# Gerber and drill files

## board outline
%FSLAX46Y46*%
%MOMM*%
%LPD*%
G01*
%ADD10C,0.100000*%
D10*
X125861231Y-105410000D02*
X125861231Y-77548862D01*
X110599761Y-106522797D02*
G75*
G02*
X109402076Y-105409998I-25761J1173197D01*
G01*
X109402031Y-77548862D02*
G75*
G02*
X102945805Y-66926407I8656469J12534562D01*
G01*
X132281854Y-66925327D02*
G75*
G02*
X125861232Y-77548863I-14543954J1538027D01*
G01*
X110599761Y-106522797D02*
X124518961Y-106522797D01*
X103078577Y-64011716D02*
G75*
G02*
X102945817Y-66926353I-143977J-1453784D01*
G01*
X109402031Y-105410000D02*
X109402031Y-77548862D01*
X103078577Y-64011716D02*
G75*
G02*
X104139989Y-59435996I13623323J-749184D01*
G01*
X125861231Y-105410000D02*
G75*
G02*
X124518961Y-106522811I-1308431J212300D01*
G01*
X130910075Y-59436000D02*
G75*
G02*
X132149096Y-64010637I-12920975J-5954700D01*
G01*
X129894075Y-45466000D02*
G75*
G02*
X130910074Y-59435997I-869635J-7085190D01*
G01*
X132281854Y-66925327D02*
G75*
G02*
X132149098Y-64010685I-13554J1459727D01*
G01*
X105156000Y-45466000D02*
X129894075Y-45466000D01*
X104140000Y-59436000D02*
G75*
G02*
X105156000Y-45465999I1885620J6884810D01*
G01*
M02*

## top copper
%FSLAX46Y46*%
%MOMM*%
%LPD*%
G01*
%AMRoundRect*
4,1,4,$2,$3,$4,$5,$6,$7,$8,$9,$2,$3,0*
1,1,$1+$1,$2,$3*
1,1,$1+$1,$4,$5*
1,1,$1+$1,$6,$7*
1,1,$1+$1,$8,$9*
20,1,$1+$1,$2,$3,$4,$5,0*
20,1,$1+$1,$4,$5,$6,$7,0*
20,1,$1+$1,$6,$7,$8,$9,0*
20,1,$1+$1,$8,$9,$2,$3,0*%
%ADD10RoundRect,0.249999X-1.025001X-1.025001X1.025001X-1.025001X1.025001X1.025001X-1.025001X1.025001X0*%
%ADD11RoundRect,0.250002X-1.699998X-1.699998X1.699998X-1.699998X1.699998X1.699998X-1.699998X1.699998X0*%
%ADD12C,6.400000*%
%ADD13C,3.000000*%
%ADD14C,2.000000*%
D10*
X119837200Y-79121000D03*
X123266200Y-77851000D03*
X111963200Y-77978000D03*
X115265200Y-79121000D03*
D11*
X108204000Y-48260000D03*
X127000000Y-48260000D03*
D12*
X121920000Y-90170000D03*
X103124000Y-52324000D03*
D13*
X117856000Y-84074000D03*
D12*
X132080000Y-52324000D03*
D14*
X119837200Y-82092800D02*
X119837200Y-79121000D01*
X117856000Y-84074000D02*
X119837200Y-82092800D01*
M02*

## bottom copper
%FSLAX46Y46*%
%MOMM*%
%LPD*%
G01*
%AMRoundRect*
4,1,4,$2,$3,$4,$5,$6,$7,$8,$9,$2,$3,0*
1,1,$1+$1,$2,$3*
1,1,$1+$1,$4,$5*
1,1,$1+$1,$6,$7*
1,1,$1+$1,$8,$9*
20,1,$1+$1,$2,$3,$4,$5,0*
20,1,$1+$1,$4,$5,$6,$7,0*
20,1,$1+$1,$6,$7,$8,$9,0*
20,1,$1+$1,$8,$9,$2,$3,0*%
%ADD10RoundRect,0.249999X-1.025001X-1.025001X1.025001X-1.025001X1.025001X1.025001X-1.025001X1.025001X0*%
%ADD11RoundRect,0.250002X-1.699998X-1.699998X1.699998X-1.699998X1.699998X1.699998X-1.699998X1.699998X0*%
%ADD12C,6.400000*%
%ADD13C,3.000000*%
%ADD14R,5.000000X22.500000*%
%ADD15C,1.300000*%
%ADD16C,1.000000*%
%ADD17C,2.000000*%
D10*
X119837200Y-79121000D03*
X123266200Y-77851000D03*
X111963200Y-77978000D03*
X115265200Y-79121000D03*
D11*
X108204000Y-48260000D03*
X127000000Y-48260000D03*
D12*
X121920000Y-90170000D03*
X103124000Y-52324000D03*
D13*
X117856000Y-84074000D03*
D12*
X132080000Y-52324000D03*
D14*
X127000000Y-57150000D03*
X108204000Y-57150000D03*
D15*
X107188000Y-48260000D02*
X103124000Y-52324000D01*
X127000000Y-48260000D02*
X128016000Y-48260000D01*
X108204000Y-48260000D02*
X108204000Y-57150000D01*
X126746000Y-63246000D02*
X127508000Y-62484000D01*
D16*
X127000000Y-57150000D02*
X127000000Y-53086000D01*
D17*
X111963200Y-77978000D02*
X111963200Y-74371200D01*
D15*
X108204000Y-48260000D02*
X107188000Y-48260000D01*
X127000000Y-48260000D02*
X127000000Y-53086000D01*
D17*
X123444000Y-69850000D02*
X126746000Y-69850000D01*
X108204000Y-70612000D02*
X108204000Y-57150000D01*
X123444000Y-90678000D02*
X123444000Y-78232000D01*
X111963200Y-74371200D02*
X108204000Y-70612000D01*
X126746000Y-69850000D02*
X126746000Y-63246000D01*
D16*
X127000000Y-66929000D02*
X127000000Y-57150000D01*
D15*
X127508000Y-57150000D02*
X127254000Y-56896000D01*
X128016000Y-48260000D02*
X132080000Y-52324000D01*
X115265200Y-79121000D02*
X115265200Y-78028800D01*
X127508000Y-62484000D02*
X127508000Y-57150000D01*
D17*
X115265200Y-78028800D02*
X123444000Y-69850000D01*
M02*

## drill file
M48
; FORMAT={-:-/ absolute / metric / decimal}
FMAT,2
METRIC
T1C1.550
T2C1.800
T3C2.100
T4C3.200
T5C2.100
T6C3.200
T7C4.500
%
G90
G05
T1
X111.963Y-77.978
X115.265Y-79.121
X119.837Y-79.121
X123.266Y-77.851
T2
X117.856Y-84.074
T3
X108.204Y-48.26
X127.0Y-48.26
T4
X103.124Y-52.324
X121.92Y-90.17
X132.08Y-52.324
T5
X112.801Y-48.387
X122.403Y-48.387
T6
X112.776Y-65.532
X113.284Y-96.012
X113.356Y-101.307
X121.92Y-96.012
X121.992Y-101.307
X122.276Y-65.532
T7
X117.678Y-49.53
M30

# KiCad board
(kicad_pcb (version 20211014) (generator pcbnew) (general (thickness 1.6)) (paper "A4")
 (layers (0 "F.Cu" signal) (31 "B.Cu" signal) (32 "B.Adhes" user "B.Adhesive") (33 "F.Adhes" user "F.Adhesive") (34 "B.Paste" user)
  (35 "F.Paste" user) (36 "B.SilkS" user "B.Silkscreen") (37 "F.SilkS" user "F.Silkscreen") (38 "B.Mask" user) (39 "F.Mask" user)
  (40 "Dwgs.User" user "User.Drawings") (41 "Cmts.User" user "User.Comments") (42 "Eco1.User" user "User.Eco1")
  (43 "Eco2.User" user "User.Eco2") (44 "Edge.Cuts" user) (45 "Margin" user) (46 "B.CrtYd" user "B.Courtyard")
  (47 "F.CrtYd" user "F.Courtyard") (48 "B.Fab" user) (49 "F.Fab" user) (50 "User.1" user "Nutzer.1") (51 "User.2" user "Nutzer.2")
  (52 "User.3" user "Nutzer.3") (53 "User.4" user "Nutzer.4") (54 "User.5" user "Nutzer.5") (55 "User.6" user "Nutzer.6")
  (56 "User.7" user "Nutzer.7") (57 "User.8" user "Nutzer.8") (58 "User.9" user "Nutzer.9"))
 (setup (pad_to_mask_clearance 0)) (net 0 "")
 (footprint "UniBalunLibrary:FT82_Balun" (layer "F.Cu") (at 117.602 65.532)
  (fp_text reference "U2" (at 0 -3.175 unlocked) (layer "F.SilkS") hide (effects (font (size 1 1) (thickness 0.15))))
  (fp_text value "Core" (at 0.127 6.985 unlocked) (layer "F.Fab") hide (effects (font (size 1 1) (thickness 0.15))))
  (pad "" np_thru_hole circle (at -4.826 0) (size 3.2 3.2) (drill 3.2) (layers *.Cu *.Mask))
  (pad "" np_thru_hole circle (at 4.6736 0) (size 3.2 3.2) (drill 3.2) (layers *.Cu *.Mask))
  (pad "1" thru_hole roundrect (at 2.2352 13.589) (size 2.55 2.55) (drill 1.55) (layers *.Cu *.Mask) (roundrect_rratio 0.09803882353))
  (pad "2" thru_hole roundrect (at 5.6642 12.319) (size 2.55 2.55) (drill 1.55) (layers *.Cu *.Mask) (roundrect_rratio 0.09803882353))
  (pad "3" thru_hole roundrect (at -5.6388 12.446) (size 2.55 2.55) (drill 1.55) (layers *.Cu *.Mask) (roundrect_rratio 0.09803882353))
  (pad "4" thru_hole roundrect (at -2.3368 13.589) (size 2.55 2.55) (drill 1.55) (layers *.Cu *.Mask) (roundrect_rratio 0.09803882353)))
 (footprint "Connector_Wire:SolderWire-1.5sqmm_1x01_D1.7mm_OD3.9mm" (layer "F.Cu") (at 108.204 48.26)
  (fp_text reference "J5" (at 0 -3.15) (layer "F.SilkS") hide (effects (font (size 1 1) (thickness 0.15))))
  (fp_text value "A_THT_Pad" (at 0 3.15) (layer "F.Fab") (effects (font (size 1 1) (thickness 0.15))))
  (pad "1" thru_hole roundrect (at 0 0) (size 3.9 3.9) (drill 2.1) (layers *.Cu *.Mask) (roundrect_rratio 0.06410307692)))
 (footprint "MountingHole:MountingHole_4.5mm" (layer "F.Cu") (at 117.6782 49.53)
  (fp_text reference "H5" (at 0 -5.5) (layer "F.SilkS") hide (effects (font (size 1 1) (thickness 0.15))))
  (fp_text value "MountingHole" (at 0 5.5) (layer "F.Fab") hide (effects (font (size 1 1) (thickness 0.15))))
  (pad "" np_thru_hole circle (at 0 0) (size 4.5 4.5) (drill 4.5) (layers *.Cu *.Mask)))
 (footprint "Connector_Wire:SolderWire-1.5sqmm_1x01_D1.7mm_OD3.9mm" (layer "F.Cu") (at 127 48.26)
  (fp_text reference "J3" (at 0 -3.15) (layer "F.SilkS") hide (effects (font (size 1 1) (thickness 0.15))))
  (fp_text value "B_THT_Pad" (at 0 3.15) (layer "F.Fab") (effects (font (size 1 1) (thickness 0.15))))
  (pad "1" thru_hole roundrect (at 0 0) (size 3.9 3.9) (drill 2.1) (layers *.Cu *.Mask) (roundrect_rratio 0.06410307692)))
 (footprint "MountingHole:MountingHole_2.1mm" (layer "F.Cu") (at 112.8014 48.387)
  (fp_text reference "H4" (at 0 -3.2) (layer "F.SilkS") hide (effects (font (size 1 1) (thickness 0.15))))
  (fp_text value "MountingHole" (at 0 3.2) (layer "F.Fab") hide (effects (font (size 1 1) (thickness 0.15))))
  (pad "" np_thru_hole circle (at 0 0) (size 2.1 2.1) (drill 2.1) (layers *.Cu *.Mask)))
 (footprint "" (layer "F.Cu") (at 121.92 90.17)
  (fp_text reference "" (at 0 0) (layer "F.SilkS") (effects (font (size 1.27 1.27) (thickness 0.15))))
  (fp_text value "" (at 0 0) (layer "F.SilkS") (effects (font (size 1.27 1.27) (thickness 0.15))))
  (pad "1" thru_hole circle (at 0 0) (size 6.4 6.4) (drill 3.2) (layers *.Cu *.Mask)))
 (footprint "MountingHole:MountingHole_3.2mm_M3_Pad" (layer "F.Cu") (at 103.124 52.324)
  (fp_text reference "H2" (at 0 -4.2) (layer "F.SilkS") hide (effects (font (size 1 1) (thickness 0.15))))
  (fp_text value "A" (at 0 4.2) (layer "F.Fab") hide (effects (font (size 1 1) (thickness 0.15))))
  (pad "1" thru_hole circle (at 0 0) (size 6.4 6.4) (drill 3.2) (layers *.Cu *.Mask)))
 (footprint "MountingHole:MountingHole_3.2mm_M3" (layer "F.Cu") (at 121.991969 101.306569)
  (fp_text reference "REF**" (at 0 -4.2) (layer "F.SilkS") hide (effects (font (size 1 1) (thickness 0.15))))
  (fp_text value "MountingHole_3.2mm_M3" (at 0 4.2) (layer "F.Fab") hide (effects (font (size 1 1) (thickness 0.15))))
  (pad "" np_thru_hole circle (at 0 0) (size 3.2 3.2) (drill 3.2) (layers *.Cu *.Mask)))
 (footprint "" (layer "F.Cu") (at 117.856 84.074)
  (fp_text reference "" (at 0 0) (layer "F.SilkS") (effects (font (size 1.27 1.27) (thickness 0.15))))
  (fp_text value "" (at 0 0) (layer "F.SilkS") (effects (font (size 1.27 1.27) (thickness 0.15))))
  (pad "1" thru_hole circle (at 0 0) (size 3 3) (drill 1.8) (layers *.Cu *.Mask)))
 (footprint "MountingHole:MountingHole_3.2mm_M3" (layer "F.Cu") (at 113.284 96.012)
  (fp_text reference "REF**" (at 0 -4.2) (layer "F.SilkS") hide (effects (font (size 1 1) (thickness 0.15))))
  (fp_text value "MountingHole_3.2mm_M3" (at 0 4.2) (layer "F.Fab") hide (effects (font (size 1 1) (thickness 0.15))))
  (pad "" np_thru_hole circle (at 0 0) (size 3.2 3.2) (drill 3.2) (layers *.Cu *.Mask)))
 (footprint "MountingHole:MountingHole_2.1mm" (layer "F.Cu") (at 122.4026 48.387)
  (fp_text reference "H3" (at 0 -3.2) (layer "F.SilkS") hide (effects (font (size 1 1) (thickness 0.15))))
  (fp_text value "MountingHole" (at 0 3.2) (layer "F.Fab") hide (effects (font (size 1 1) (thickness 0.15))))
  (pad "" np_thru_hole circle (at 0 0) (size 2.1 2.1) (drill 2.1) (layers *.Cu *.Mask)))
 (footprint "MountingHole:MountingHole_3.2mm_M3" (layer "F.Cu") (at 113.355969 101.306569)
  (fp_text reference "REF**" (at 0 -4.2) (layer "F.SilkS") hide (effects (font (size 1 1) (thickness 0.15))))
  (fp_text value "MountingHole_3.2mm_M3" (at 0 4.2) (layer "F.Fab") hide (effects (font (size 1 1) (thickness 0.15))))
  (pad "" np_thru_hole circle (at 0 0) (size 3.2 3.2) (drill 3.2) (layers *.Cu *.Mask)))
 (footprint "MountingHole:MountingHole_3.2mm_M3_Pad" (layer "F.Cu") (at 132.08 52.324)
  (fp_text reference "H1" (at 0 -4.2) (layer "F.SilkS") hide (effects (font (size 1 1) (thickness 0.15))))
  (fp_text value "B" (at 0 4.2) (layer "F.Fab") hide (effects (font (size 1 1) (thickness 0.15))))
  (pad "1" thru_hole circle (at 0 0) (size 6.4 6.4) (drill 3.2) (layers *.Cu *.Mask)))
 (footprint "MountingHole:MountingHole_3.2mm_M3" (layer "F.Cu") (at 121.92 96.012)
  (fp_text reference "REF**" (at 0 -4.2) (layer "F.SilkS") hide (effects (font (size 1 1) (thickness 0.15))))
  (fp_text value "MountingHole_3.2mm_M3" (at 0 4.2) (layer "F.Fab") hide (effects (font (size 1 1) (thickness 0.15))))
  (pad "" np_thru_hole circle (at 0 0) (size 3.2 3.2) (drill 3.2) (layers *.Cu *.Mask)))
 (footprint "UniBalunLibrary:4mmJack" (layer "B.Cu") (at 127.254 56.896 90)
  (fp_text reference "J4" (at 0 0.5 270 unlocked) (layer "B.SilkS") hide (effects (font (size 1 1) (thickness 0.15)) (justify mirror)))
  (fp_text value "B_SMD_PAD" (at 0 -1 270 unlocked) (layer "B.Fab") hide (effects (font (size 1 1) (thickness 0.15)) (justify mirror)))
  (pad "1" smd rect (at -0.254 -0.254 90) (size 22.5 5) (layers "B.Cu" "B.Mask")))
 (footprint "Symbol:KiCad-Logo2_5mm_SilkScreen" (layer "B.Cu") (at 117.729 58.547 180)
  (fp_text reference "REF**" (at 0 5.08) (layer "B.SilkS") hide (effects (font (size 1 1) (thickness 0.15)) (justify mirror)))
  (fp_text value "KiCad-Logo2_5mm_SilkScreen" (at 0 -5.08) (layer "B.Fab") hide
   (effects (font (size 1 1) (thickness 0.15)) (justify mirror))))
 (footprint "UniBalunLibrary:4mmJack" (layer "B.Cu") (at 108.458 56.896 90)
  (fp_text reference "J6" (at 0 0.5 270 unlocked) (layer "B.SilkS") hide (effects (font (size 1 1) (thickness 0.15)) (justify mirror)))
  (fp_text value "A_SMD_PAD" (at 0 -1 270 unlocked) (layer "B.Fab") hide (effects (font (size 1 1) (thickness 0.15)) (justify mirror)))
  (pad "1" smd rect (at -0.254 -0.254 90) (size 22.5 5) (layers "B.Cu" "B.Mask")))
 (gr_line (start 125.861231 105.41) (end 125.861231 77.548862) (layer "Edge.Cuts") (width 0.1))
 (gr_arc (start 110.599761 106.522797) (mid 109.77522 106.209299) (end 109.402031 105.41) (layer "Edge.Cuts") (width 0.1))
 (gr_arc (start 109.402031 77.548862) (mid 105.04112 72.92614) (end 102.945817 66.926406) (layer "Edge.Cuts") (width 0.1))
 (gr_arc (start 132.281854 66.925327) (mid 130.254542 72.952072) (end 125.861231 77.548862) (layer "Edge.Cuts") (width 0.1))
 (gr_line (start 110.599761 106.522797) (end 124.518961 106.522797) (layer "Edge.Cuts") (width 0.1))
 (gr_arc (start 103.078577 64.011716) (mid 104.394 65.532) (end 102.945817 66.926406) (layer "Edge.Cuts") (width 0.1))
 (gr_line (start 109.402031 105.41) (end 109.402031 77.548862) (layer "Edge.Cuts") (width 0.1))
 (gr_arc (start 103.078577 64.011716) (mid 103.410896 61.677837) (end 104.14 59.436) (layer "Edge.Cuts") (width 0.1))
 (gr_arc (start 125.861231 105.41) (mid 125.398804 106.218144) (end 124.518961 106.522797) (layer "Edge.Cuts") (width 0.1))
 (gr_arc (start 130.910075 59.436) (mid 131.721418 61.671361) (end 132.149094 64.010637) (layer "Edge.Cuts") (width 0.1))
 (gr_arc (start 129.894075 45.466) (mid 136.144 52.033405) (end 130.910075 59.436) (layer "Edge.Cuts") (width 0.1))
 (gr_arc (start 132.281854 66.925327) (mid 130.81 65.532) (end 132.149094 64.010637) (layer "Edge.Cuts") (width 0.1))
 (gr_line (start 105.156 45.466) (end 129.894075 45.466) (layer "Edge.Cuts") (width 0.1))
 (gr_arc (start 104.14 59.436) (mid 98.906069 52.033405) (end 105.156 45.466) (layer "Edge.Cuts") (width 0.1))
 (segment (start 119.8372 82.0928) (end 119.8372 79.121) (width 2) (layer "F.Cu") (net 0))
 (segment (start 117.856 84.074) (end 119.8372 82.0928) (width 2) (layer "F.Cu") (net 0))
 (segment (start 107.188 48.26) (end 103.124 52.324) (width 1.3) (layer "B.Cu") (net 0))
 (segment (start 127 48.26) (end 128.016 48.26) (width 1.3) (layer "B.Cu") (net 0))
 (segment (start 108.204 48.26) (end 108.204 57.15) (width 1.3) (layer "B.Cu") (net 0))
 (segment (start 126.746 63.246) (end 127.508 62.484) (width 1.3) (layer "B.Cu") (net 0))
 (segment (start 127 57.15) (end 127 53.086) (width 1) (layer "B.Cu") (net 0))
 (segment (start 111.9632 77.978) (end 111.9632 74.3712) (width 2) (layer "B.Cu") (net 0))
 (segment (start 108.204 48.26) (end 107.188 48.26) (width 1.3) (layer "B.Cu") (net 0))
 (segment (start 127 48.26) (end 127 53.086) (width 1.3) (layer "B.Cu") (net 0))
 (segment (start 123.444 69.85) (end 126.746 69.85) (width 2) (layer "B.Cu") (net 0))
 (segment (start 108.204 70.612) (end 108.204 57.15) (width 2) (layer "B.Cu") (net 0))
 (segment (start 123.444 90.678) (end 123.444 78.232) (width 2) (layer "B.Cu") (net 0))
 (segment (start 111.9632 74.3712) (end 108.204 70.612) (width 2) (layer "B.Cu") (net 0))
 (segment (start 126.746 69.85) (end 126.746 63.246) (width 2) (layer "B.Cu") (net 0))
 (segment (start 127 66.929) (end 127 57.15) (width 1) (layer "B.Cu") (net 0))
 (segment (start 127.508 57.15) (end 127.254 56.896) (width 1.3) (layer "B.Cu") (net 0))
 (segment (start 128.016 48.26) (end 132.08 52.324) (width 1.3) (layer "B.Cu") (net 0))
 (segment (start 115.2652 79.121) (end 115.2652 78.0288) (width 1.3) (layer "B.Cu") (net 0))
 (segment (start 127.508 62.484) (end 127.508 57.15) (width 1.3) (layer "B.Cu") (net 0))
 (segment (start 115.2652 78.0288) (end 123.444 69.85) (width 2) (layer "B.Cu") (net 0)))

